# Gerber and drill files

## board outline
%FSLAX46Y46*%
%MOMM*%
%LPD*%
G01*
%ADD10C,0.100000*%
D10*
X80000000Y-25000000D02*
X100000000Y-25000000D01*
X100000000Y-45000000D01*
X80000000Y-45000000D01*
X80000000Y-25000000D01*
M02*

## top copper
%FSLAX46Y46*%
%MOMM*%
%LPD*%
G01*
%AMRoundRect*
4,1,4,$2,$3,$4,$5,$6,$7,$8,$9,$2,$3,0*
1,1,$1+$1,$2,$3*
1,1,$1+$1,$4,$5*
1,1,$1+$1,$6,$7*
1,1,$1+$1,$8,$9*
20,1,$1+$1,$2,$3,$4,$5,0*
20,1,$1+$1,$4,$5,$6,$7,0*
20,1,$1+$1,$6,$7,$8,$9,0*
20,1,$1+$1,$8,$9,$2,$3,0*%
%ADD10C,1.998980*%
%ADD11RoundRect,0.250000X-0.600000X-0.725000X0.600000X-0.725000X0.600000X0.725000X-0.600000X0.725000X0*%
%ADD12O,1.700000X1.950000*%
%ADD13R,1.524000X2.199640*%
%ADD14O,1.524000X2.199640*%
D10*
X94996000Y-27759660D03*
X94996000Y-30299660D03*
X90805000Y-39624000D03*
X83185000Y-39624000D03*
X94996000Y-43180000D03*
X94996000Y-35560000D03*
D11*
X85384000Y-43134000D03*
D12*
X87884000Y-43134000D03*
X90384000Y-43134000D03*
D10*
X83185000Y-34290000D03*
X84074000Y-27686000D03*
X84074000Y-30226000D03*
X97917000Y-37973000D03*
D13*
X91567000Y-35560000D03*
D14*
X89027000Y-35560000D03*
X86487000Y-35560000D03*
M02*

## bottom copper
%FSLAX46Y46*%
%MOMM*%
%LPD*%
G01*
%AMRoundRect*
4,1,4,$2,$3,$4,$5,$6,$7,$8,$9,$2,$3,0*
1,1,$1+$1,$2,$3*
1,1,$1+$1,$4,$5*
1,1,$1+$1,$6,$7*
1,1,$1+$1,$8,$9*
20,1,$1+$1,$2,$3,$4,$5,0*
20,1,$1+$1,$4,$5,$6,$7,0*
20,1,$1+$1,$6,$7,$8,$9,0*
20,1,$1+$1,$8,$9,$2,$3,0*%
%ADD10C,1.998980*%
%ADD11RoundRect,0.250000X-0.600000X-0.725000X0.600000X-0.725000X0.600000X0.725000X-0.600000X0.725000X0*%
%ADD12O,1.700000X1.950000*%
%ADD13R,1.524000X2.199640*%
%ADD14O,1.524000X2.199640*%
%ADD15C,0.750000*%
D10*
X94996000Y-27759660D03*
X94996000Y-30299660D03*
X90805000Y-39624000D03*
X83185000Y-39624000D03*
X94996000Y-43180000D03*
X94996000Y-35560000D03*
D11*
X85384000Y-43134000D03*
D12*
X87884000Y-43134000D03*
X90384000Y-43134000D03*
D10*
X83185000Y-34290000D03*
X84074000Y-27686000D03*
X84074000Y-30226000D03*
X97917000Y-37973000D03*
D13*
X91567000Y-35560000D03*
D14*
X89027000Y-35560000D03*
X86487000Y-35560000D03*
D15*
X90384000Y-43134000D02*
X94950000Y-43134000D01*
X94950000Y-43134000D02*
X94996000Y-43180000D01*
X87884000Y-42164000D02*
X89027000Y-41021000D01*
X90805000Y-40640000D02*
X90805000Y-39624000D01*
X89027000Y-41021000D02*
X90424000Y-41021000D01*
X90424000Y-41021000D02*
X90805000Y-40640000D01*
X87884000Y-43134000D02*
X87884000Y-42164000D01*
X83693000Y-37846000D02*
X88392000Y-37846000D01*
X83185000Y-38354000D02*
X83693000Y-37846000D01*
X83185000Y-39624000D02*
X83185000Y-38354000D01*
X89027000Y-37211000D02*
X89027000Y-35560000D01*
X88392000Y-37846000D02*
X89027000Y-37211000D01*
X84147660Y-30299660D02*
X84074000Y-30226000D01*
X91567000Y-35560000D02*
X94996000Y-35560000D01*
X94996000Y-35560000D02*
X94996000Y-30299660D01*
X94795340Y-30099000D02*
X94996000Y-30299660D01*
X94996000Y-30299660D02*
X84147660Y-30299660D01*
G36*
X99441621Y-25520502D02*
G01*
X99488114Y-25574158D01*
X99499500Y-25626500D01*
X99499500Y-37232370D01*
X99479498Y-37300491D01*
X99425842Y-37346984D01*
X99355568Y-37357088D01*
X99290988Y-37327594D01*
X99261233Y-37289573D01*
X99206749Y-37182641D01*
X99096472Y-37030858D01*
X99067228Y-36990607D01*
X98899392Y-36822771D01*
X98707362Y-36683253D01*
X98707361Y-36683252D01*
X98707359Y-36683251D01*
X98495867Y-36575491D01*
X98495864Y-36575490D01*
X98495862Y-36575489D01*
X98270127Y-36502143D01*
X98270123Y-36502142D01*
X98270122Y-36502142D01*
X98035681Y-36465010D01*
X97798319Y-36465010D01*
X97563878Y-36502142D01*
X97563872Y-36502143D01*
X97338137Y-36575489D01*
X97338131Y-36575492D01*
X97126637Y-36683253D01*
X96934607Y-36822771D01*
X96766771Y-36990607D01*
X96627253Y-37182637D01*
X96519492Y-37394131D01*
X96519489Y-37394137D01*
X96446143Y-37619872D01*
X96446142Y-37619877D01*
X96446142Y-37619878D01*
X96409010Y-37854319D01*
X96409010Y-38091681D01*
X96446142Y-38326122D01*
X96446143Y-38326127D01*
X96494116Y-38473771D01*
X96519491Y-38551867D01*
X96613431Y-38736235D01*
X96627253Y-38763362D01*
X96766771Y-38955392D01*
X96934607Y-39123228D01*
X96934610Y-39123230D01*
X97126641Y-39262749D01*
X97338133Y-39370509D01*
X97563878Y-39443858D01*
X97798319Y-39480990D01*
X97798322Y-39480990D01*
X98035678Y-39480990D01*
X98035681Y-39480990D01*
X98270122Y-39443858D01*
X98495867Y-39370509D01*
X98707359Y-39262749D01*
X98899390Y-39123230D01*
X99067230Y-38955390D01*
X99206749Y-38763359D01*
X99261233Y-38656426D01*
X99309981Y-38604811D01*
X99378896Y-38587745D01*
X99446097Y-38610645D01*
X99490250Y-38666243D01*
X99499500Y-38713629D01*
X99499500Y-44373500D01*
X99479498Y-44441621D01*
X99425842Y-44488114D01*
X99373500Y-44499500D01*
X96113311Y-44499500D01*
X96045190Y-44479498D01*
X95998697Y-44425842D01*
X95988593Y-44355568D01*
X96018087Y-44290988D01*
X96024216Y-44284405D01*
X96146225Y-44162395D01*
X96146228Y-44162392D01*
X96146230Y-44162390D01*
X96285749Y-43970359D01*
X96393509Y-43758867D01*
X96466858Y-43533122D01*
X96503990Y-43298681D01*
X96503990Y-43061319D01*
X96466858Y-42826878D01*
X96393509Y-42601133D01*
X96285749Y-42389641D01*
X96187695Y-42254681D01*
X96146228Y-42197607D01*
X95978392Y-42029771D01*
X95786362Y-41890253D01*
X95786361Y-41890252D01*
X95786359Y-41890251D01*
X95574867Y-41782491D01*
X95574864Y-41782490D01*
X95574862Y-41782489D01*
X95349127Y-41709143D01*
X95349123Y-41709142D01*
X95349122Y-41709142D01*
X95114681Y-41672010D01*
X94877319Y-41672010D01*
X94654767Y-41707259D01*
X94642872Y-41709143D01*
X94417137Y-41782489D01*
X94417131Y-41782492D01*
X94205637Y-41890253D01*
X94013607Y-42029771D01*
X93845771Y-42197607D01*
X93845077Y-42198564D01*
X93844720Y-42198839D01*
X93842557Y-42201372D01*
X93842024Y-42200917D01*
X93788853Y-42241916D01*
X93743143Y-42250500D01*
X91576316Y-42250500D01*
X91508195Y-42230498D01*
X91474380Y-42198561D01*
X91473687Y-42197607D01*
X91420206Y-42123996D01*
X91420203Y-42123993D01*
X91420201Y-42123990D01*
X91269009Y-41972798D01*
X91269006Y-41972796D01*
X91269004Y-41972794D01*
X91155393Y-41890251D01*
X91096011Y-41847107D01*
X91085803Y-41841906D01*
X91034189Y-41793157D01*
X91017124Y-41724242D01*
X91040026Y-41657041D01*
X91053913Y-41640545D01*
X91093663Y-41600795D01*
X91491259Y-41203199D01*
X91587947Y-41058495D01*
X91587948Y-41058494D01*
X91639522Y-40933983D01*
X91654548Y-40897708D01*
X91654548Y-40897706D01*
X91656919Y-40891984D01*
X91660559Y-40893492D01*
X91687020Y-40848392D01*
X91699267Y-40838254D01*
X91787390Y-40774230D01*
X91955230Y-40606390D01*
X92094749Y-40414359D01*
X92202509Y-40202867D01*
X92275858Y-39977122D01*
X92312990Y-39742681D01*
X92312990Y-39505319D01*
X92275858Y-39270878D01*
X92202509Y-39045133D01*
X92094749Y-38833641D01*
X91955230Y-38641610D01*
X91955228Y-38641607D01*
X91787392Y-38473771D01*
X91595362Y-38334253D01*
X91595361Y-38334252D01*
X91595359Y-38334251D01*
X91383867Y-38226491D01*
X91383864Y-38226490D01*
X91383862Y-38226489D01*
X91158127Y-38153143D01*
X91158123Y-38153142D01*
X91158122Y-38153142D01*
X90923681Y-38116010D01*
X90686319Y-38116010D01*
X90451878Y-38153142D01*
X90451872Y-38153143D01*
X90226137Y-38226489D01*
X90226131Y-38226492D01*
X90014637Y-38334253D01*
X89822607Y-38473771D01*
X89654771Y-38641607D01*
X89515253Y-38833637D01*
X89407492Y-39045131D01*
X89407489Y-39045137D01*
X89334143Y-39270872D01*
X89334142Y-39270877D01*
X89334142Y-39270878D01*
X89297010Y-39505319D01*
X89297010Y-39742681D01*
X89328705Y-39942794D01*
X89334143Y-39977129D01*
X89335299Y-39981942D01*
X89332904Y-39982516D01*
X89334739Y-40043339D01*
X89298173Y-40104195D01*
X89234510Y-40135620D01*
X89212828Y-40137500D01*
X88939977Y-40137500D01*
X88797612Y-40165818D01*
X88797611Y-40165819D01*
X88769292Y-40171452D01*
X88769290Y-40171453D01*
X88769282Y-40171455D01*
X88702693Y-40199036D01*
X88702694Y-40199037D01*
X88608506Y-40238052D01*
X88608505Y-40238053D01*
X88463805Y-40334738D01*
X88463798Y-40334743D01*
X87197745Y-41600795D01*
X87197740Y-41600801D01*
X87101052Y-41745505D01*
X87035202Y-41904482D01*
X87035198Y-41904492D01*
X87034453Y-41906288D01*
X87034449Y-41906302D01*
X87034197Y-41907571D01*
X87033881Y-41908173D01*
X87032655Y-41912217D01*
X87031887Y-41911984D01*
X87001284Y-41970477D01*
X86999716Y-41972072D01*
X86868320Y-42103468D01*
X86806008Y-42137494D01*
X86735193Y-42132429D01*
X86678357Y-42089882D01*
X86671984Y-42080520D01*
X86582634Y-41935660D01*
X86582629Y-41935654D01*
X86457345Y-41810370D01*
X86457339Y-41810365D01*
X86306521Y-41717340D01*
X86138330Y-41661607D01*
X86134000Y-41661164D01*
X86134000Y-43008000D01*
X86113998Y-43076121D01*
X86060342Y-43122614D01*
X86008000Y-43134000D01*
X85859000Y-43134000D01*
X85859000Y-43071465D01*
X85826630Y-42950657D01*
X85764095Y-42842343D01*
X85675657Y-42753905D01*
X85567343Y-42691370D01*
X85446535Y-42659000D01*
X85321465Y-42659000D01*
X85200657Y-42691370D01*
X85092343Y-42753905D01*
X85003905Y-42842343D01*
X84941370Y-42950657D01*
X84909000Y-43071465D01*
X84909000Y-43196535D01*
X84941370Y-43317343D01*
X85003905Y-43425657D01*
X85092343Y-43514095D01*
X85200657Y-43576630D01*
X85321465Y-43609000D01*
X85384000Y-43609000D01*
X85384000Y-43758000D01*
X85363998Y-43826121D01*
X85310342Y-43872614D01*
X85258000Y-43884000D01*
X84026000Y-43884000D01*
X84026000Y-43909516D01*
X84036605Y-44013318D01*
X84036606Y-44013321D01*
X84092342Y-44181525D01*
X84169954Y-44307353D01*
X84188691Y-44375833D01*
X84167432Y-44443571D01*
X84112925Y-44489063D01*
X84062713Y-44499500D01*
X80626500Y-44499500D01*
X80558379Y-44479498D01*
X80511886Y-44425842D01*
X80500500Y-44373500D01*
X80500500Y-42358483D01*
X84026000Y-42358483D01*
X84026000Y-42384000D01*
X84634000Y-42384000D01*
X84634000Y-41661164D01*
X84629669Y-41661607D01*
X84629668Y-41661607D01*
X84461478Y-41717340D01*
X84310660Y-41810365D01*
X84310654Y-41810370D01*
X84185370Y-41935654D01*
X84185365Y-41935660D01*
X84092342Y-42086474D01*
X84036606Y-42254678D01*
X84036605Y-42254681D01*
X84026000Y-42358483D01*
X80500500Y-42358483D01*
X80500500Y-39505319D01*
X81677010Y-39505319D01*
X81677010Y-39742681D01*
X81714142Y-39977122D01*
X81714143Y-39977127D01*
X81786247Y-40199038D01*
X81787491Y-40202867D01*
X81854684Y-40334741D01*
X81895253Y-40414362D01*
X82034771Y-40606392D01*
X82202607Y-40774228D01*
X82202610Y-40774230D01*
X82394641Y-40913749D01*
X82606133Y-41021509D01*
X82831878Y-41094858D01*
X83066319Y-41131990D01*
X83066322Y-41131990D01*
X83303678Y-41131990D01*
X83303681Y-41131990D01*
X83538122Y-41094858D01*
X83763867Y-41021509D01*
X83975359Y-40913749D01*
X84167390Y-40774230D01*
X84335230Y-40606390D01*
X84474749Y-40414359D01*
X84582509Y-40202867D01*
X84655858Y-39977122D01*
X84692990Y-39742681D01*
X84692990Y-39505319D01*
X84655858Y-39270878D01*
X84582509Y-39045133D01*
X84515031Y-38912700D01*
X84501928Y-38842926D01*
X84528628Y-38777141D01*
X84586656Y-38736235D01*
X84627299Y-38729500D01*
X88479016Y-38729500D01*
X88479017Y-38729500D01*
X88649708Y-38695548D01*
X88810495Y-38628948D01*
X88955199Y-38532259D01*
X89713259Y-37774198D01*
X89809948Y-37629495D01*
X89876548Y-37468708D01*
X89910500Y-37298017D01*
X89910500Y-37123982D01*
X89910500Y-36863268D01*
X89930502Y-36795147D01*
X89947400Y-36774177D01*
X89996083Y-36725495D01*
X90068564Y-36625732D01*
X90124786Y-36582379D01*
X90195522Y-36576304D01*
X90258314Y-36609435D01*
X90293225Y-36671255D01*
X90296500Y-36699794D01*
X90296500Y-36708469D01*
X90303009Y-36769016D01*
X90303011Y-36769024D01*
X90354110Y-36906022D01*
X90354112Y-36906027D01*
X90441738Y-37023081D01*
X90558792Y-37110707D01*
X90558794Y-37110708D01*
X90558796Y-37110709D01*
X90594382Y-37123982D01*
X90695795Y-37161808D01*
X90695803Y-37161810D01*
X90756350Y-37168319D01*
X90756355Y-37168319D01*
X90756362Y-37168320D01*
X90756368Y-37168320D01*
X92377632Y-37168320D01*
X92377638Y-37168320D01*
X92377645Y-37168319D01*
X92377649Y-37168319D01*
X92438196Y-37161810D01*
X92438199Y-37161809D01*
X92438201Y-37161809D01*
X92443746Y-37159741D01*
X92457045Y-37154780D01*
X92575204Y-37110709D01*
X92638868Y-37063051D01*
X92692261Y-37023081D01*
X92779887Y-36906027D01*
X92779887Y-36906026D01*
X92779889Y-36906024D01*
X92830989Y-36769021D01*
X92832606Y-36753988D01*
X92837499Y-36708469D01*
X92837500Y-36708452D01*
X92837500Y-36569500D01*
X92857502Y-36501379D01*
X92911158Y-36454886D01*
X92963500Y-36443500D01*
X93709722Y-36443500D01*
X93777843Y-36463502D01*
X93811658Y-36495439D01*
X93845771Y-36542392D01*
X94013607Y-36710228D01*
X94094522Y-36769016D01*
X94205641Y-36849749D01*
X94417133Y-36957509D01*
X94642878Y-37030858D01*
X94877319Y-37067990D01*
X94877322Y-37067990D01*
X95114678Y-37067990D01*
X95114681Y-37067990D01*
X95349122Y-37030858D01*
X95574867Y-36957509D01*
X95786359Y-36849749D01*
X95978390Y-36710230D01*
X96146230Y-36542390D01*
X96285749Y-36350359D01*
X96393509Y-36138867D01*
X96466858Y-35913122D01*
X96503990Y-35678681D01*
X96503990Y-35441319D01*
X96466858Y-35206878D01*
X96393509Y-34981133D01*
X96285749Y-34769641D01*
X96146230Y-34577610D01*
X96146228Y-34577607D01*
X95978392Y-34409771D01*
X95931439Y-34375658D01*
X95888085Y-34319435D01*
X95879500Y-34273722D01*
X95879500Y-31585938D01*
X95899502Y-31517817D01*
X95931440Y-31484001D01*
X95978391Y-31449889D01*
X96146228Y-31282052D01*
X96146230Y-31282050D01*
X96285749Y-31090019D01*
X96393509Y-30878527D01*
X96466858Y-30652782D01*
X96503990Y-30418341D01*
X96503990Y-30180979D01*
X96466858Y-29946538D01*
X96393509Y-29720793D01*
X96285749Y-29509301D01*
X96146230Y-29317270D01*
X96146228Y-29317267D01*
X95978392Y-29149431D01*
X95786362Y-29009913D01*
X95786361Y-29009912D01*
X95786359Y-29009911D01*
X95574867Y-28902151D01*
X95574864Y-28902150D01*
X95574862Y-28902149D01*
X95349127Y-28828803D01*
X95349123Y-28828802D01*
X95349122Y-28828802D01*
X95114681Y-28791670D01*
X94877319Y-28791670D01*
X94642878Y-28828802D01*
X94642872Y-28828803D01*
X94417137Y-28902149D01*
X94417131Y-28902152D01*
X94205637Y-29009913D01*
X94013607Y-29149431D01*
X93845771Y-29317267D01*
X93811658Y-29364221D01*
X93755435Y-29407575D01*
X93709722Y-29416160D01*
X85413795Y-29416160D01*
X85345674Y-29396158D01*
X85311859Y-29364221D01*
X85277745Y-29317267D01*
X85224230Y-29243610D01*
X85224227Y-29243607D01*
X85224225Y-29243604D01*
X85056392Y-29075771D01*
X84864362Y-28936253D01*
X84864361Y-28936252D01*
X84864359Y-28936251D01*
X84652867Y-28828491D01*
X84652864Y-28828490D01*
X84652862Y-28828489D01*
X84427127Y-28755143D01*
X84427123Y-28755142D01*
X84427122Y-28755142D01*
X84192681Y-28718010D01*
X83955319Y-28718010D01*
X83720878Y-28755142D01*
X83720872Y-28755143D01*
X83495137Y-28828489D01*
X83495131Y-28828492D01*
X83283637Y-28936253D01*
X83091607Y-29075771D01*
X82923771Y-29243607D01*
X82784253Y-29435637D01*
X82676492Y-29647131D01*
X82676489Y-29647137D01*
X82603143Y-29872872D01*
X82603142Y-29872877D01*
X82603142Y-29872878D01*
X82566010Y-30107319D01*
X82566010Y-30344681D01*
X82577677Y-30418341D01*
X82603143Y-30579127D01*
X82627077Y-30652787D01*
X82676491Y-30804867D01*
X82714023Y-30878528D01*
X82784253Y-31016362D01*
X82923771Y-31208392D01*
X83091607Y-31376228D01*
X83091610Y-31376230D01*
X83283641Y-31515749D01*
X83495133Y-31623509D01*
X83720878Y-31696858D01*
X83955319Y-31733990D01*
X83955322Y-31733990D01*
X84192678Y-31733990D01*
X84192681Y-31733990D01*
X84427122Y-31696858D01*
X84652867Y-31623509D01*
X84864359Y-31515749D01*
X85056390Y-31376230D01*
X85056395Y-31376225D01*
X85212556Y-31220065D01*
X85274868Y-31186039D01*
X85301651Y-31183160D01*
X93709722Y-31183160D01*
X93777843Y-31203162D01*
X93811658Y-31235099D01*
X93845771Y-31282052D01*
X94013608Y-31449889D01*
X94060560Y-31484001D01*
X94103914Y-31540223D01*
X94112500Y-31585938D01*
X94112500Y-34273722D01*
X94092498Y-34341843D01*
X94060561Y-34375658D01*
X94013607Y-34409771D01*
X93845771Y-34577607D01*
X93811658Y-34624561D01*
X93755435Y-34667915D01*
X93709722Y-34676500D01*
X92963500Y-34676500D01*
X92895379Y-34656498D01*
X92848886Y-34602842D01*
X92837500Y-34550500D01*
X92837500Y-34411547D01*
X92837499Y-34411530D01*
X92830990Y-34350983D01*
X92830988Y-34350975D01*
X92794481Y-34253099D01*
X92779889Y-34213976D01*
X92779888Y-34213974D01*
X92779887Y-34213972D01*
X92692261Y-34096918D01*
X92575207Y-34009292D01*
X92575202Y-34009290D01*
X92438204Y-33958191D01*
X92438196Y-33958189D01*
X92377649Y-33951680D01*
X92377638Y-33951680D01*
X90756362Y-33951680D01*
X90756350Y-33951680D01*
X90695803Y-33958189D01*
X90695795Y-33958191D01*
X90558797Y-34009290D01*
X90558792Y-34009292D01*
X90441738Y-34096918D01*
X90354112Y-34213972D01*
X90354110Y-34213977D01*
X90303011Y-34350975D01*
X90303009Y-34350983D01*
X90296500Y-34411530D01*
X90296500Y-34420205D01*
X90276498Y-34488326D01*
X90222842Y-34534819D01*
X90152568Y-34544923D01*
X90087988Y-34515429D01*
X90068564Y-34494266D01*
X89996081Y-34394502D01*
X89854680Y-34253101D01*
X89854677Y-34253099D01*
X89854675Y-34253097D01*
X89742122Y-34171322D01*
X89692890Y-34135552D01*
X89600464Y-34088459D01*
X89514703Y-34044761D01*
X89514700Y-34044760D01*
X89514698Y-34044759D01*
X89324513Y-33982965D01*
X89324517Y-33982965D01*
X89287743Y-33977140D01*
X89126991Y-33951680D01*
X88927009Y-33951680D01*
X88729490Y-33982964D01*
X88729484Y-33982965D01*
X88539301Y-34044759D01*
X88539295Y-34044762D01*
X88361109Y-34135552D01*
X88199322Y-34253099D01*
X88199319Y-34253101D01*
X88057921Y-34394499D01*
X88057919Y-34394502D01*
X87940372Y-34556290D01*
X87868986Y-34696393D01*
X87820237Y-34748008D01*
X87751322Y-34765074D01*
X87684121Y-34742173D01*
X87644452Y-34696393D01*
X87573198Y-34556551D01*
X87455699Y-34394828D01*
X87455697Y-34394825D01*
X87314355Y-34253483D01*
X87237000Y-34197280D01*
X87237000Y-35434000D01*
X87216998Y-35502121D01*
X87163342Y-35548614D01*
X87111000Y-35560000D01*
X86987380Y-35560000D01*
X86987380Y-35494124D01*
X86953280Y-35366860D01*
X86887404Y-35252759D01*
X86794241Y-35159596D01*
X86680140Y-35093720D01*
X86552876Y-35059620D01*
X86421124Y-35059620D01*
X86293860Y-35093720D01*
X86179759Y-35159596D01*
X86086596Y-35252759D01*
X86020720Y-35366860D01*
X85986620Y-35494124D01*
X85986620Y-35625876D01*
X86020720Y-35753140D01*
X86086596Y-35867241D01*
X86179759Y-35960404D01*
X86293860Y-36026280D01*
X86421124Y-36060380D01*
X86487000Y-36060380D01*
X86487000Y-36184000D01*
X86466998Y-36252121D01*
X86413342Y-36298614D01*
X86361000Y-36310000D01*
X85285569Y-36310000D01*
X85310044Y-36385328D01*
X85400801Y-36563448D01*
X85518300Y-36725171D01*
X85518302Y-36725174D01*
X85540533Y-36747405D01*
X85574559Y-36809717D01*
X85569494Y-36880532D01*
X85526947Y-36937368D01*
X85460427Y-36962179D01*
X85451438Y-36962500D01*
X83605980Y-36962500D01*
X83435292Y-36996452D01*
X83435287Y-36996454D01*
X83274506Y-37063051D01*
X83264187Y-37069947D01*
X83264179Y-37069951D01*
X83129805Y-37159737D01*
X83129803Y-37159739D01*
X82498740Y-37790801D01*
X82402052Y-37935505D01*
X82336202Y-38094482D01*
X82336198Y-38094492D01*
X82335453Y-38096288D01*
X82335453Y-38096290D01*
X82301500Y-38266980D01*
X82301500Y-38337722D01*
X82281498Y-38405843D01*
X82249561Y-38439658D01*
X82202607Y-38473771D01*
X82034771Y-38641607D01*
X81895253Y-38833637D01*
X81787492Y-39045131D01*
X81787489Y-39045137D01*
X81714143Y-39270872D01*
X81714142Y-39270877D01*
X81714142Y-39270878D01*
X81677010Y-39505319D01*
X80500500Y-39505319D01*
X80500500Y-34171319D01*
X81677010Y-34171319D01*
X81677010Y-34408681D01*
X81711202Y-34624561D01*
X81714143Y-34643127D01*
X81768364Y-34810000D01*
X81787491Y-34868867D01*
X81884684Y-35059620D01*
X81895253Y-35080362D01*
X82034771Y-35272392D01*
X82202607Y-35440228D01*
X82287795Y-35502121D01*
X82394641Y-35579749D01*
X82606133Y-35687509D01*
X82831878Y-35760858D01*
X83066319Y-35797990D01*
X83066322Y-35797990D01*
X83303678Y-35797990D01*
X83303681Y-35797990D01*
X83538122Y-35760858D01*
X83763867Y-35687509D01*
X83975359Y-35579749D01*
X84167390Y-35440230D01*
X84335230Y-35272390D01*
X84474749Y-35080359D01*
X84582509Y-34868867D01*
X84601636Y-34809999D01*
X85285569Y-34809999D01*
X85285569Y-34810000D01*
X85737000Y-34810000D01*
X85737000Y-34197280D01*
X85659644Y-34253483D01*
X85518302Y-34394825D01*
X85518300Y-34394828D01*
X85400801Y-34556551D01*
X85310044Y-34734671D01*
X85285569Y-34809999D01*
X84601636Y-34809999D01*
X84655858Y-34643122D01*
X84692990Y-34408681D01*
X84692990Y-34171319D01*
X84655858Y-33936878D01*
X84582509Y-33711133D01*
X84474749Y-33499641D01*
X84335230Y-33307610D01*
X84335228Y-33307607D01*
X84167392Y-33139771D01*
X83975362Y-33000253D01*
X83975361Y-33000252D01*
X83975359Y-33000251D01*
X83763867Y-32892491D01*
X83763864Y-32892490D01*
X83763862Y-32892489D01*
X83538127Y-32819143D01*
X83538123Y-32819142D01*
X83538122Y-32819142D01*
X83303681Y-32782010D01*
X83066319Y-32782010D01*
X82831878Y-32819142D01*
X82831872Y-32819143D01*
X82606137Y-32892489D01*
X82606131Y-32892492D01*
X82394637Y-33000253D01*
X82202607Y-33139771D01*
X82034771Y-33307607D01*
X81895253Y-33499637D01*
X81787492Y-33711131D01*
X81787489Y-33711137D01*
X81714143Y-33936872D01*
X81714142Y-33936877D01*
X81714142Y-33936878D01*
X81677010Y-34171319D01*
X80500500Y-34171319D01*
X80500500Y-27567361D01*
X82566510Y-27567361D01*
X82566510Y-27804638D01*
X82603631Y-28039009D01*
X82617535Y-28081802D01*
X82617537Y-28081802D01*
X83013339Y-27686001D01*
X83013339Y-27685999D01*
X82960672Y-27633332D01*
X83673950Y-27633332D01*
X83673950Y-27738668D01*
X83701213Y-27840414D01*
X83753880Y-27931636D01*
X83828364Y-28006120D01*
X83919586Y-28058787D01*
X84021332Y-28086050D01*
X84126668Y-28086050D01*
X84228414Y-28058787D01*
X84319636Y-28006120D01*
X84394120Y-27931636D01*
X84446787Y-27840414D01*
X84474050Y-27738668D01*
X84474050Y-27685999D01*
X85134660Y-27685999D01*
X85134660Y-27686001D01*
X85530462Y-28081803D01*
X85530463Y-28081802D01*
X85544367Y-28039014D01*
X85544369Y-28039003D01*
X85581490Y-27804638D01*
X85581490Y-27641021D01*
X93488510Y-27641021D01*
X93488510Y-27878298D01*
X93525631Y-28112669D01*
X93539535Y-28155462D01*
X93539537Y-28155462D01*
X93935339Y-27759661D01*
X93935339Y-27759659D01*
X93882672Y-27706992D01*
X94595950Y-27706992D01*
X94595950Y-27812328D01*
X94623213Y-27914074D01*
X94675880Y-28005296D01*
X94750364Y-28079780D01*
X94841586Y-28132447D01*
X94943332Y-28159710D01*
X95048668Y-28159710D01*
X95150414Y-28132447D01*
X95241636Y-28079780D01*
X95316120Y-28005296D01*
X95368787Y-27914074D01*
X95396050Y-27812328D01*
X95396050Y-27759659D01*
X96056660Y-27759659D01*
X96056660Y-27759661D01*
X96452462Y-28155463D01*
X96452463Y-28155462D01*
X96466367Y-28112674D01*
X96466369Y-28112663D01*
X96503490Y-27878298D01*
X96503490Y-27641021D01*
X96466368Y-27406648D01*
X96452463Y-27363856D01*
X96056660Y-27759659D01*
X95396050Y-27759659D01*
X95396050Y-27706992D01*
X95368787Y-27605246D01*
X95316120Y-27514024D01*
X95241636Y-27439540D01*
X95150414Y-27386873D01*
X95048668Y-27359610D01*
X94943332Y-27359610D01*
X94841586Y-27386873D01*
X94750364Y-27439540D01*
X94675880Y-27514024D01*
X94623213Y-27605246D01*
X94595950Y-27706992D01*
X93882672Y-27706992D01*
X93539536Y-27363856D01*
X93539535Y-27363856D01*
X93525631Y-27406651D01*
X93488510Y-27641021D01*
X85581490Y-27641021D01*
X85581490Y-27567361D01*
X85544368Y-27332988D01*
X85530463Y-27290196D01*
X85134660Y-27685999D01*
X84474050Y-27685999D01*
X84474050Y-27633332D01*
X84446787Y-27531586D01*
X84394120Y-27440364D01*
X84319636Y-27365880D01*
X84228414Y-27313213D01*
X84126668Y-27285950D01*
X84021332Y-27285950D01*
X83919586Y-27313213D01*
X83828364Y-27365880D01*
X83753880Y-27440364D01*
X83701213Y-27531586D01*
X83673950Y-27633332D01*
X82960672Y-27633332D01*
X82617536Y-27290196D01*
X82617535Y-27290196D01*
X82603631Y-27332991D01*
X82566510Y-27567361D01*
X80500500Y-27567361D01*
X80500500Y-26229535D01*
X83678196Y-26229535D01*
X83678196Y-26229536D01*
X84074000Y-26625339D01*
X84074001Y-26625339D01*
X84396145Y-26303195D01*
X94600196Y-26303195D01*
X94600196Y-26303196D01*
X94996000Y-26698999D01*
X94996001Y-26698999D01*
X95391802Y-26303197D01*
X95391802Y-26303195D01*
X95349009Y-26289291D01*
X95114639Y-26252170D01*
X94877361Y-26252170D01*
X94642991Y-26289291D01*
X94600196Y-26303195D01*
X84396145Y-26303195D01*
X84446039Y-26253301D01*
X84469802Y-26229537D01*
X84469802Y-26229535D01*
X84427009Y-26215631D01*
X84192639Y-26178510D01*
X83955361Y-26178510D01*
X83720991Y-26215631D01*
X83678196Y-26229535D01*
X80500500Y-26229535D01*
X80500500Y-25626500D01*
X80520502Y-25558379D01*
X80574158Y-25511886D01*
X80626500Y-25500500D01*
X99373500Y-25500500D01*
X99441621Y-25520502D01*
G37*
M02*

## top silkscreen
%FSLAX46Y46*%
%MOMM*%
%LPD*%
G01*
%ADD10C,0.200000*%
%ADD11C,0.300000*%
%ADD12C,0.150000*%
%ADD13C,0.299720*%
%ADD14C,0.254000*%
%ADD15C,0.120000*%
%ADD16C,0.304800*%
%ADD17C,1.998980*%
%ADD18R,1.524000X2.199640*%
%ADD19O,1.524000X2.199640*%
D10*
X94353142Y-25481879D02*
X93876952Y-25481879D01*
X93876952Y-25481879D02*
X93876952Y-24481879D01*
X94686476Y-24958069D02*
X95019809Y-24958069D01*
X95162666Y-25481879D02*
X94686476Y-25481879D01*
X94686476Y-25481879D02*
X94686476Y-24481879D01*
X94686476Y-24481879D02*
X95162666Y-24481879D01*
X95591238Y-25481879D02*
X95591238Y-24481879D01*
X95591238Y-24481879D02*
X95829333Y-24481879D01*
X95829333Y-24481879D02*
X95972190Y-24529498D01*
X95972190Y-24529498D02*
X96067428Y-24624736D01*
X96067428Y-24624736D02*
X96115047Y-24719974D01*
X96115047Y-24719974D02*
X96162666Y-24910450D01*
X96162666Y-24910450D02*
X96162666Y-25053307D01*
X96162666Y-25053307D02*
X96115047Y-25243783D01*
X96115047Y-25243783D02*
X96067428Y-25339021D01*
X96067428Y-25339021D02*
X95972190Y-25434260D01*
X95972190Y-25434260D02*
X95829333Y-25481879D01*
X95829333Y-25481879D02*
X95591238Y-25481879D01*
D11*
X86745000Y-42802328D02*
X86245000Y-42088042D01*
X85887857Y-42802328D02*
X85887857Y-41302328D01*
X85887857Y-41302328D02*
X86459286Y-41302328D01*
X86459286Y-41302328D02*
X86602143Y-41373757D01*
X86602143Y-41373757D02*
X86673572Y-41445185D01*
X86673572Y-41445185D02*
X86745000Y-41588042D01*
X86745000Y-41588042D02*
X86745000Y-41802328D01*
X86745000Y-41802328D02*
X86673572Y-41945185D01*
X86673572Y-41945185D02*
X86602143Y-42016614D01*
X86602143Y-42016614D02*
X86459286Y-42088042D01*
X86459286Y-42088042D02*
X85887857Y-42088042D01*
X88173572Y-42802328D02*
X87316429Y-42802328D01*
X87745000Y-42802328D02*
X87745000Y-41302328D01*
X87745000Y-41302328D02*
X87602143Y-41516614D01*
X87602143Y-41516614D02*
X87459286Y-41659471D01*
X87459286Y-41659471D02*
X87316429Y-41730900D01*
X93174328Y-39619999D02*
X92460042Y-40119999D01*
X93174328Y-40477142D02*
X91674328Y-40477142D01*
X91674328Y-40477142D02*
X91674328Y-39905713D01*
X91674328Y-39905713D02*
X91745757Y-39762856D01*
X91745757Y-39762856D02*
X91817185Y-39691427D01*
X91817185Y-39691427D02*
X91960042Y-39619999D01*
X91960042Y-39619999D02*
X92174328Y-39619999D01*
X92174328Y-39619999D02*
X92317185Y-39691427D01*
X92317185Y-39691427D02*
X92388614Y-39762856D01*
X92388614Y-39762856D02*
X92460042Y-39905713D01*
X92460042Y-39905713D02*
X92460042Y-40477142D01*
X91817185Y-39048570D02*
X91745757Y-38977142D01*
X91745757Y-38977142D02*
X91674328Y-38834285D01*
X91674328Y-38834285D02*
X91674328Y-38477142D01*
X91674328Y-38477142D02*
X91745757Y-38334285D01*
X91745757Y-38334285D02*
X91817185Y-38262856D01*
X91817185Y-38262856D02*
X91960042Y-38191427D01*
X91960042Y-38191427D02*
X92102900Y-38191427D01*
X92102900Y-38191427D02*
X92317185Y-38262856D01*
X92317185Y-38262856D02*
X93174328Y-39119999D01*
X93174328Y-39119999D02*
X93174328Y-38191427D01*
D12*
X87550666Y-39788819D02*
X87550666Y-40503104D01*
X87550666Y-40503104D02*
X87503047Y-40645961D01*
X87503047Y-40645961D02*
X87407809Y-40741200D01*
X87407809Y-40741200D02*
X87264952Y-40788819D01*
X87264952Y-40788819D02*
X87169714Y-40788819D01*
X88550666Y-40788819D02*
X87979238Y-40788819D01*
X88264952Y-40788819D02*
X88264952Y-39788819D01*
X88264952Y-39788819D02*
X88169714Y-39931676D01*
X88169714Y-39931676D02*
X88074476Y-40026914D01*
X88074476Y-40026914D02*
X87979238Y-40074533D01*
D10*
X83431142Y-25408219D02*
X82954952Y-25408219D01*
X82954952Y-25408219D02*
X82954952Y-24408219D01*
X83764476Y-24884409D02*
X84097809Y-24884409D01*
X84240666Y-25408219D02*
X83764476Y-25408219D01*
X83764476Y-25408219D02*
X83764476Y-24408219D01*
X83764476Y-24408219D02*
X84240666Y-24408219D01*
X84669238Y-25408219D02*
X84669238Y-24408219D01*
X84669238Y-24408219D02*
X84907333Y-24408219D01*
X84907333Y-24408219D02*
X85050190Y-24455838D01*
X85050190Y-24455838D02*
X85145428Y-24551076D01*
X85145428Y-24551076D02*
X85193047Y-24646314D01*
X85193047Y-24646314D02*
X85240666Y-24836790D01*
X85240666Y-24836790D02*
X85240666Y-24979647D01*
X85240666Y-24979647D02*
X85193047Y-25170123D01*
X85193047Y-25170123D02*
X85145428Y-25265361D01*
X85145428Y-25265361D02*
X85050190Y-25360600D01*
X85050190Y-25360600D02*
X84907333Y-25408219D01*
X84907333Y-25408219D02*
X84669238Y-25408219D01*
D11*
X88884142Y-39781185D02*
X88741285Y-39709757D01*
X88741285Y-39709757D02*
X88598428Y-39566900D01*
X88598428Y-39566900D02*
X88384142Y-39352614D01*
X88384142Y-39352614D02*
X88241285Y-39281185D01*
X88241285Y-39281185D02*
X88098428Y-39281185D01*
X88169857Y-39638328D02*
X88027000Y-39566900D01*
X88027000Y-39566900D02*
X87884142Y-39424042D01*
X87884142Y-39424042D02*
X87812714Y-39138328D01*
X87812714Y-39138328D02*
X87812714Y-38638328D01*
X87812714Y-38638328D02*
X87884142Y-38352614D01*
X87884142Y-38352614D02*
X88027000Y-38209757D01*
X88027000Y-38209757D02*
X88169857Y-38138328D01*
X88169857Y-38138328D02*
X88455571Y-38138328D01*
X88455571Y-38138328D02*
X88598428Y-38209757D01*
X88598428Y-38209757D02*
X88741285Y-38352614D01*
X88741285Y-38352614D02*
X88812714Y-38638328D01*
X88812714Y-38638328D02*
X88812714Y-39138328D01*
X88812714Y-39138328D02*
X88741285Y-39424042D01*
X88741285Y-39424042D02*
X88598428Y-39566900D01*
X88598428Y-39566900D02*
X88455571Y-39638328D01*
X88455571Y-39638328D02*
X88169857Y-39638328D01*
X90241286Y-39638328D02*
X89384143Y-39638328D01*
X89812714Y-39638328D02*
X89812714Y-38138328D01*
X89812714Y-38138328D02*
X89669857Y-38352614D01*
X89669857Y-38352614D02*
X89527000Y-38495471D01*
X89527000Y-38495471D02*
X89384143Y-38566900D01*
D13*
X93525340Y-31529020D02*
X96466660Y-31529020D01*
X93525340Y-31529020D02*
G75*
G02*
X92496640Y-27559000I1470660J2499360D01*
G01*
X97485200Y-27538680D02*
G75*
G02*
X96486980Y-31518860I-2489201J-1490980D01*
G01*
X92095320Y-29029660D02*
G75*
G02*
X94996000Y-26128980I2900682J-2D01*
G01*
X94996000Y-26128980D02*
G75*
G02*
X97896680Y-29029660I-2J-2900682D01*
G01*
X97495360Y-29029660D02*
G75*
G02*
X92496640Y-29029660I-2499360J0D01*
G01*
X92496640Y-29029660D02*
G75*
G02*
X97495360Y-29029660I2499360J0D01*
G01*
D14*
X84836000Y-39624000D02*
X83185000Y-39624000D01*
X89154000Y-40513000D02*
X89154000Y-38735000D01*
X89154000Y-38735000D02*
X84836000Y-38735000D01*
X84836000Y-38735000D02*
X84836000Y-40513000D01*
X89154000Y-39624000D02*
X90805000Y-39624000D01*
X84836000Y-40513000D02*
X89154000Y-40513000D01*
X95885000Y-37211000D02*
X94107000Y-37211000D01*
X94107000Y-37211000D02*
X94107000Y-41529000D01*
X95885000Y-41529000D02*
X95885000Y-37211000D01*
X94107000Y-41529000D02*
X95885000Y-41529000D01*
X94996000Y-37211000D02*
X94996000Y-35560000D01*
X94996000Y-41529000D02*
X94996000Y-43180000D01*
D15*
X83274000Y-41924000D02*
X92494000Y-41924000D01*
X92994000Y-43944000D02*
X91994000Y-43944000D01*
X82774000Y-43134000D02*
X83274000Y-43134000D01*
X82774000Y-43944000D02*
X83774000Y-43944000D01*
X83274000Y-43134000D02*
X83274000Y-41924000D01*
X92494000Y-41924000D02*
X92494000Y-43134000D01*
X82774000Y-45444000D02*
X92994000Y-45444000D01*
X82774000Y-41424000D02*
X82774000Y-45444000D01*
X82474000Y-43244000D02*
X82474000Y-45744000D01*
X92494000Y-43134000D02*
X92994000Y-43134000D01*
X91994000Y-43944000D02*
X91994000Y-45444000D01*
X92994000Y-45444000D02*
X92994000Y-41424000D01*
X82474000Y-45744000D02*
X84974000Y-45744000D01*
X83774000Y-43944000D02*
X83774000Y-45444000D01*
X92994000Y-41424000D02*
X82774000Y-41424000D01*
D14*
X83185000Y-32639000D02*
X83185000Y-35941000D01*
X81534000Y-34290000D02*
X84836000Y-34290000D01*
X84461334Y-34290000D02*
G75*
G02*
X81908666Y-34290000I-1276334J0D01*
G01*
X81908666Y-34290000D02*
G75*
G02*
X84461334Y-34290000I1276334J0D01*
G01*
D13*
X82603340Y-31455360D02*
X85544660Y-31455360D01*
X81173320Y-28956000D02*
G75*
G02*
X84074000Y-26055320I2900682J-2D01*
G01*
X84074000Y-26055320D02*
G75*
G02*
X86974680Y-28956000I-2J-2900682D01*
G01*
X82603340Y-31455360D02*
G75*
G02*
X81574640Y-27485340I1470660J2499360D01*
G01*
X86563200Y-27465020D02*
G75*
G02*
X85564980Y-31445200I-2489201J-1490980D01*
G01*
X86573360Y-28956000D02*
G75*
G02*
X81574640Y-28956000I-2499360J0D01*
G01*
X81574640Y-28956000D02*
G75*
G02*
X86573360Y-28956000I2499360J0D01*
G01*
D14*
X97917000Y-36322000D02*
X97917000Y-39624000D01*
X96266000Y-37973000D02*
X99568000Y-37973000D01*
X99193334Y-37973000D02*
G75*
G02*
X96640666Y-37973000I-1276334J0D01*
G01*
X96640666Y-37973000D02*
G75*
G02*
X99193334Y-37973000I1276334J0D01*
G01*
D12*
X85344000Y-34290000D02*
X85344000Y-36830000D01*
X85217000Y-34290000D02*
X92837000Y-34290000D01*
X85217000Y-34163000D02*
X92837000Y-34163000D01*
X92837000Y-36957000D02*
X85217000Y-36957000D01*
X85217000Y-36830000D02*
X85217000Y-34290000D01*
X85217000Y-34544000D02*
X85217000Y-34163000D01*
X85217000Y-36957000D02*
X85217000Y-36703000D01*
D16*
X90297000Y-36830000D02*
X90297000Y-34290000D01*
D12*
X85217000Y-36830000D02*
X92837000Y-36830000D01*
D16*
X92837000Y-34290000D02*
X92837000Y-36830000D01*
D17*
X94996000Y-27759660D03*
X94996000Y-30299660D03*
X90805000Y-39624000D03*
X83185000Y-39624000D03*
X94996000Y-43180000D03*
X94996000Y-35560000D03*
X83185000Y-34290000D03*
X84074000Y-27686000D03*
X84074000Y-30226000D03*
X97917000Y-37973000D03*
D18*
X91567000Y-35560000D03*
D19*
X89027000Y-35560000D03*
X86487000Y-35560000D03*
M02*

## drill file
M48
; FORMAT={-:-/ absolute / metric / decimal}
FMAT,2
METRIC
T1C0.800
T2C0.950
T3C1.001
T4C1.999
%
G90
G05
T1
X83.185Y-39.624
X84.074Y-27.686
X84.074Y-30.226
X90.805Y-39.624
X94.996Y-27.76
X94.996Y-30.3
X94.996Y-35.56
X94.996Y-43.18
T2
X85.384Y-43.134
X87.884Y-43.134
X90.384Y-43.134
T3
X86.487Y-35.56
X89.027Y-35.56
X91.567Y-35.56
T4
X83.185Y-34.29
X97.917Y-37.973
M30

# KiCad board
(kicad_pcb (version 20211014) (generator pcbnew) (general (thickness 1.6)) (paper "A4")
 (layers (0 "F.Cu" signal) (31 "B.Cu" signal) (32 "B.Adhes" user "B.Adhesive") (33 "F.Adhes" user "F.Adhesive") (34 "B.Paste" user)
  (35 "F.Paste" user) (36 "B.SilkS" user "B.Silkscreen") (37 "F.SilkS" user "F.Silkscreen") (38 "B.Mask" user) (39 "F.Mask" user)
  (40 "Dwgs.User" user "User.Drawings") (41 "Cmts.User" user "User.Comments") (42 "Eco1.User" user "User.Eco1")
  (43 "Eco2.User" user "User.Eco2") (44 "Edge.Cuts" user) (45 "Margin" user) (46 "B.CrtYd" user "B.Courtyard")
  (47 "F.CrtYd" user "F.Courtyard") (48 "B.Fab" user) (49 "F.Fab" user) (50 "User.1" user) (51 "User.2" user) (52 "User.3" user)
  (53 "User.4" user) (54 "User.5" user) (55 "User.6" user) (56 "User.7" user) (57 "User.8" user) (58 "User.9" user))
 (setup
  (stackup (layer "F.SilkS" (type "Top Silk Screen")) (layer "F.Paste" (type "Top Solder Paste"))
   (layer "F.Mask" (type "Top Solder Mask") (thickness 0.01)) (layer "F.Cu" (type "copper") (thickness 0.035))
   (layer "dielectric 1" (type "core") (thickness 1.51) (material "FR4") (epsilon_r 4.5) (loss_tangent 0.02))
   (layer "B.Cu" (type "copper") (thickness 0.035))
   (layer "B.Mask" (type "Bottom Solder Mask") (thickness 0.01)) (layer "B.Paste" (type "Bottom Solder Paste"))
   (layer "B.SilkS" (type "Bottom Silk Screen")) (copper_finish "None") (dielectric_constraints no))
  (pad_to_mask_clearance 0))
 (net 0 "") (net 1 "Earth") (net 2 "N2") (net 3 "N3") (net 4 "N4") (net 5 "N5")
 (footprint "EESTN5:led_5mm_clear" (layer "F.Cu") (at 94.996 29.02966)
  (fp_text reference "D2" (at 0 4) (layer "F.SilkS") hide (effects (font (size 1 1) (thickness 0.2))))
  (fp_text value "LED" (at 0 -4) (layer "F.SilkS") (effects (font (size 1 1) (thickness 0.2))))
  (fp_line (start -1.47066 2.49936) (end 1.47066 2.49936) (layer "F.SilkS") (width 0.29972))
  (fp_arc (start -1.47066 2.49936) (mid -2.807228 0.727401) (end -2.49936 -1.47066) (layer "F.SilkS") (width 0.29972))
  (fp_arc (start 2.4892 -1.49098) (mid 2.814412 0.705848) (end 1.49098 2.4892) (layer "F.SilkS") (width 0.29972))
  (fp_arc (start -2.90068 0) (mid -2.05109 -2.05109) (end 0 -2.90068) (layer "F.SilkS") (width 0.29972))
  (fp_arc (start 0 -2.90068) (mid 2.05109 -2.05109) (end 2.90068 0) (layer "F.SilkS") (width 0.29972))
  (fp_circle (center 0 0) (end -2.49936 0) (layer "F.SilkS") (width 0.29972) (fill none))
  (pad "1" thru_hole circle locked (at 0 -1.27) (size 1.99898 1.99898) (drill 0.8001) (layers *.Cu *.Mask "F.SilkS") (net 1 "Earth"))
  (pad "2" thru_hole circle locked (at 0 1.27) (size 1.99898 1.99898) (drill 0.8001) (layers *.Cu *.Mask "F.SilkS") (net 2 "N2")))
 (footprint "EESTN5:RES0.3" (layer "F.Cu") (at 86.995 39.624 180) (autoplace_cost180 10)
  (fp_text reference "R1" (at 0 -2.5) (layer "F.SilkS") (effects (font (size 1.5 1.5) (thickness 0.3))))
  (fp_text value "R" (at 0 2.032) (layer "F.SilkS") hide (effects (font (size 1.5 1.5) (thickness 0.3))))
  (fp_line (start 2.159 0) (end 3.81 0) (layer "F.SilkS") (width 0.254))
  (fp_line (start -2.159 -0.889) (end -2.159 0.889) (layer "F.SilkS") (width 0.254))
  (fp_line (start -2.159 0.889) (end 2.159 0.889) (layer "F.SilkS") (width 0.254))
  (fp_line (start 2.159 0.889) (end 2.159 -0.889) (layer "F.SilkS") (width 0.254))
  (fp_line (start -2.159 0) (end -3.81 0) (layer "F.SilkS") (width 0.254))
  (fp_line (start 2.159 -0.889) (end -2.159 -0.889) (layer "F.SilkS") (width 0.254))
  (pad "1" thru_hole circle locked (at -3.81 0 180) (size 1.99898 1.99898) (drill 0.8001) (layers *.Cu *.Mask "F.SilkS") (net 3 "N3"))
  (pad "2" thru_hole circle locked (at 3.81 0 180) (size 1.99898 1.99898) (drill 0.8001) (layers *.Cu *.Mask "F.SilkS") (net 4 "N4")))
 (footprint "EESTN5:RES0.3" (layer "F.Cu") (at 94.996 39.37 90) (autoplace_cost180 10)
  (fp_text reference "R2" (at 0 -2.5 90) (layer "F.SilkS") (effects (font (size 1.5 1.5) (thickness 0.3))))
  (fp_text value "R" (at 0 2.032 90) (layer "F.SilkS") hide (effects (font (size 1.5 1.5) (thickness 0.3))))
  (fp_line (start 2.159 0.889) (end 2.159 -0.889) (layer "F.SilkS") (width 0.254))
  (fp_line (start 2.159 -0.889) (end -2.159 -0.889) (layer "F.SilkS") (width 0.254))
  (fp_line (start -2.159 0.889) (end 2.159 0.889) (layer "F.SilkS") (width 0.254))
  (fp_line (start -2.159 -0.889) (end -2.159 0.889) (layer "F.SilkS") (width 0.254))
  (fp_line (start 2.159 0) (end 3.81 0) (layer "F.SilkS") (width 0.254))
  (fp_line (start -2.159 0) (end -3.81 0) (layer "F.SilkS") (width 0.254))
  (pad "1" thru_hole circle locked (at -3.81 0 90) (size 1.99898 1.99898) (drill 0.8001) (layers *.Cu *.Mask "F.SilkS") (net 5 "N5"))
  (pad "2" thru_hole circle locked (at 3.81 0 90) (size 1.99898 1.99898) (drill 0.8001) (layers *.Cu *.Mask "F.SilkS") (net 2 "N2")))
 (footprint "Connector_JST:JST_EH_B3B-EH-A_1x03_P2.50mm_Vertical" (layer "F.Cu") (at 85.384 43.134)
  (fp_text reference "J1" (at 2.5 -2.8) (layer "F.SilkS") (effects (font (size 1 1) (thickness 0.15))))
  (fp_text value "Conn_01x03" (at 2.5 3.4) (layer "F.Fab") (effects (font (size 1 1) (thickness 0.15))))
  (fp_line (start -2.11 -1.21) (end 7.11 -1.21) (layer "F.SilkS") (width 0.12))
  (fp_line (start 7.61 0.81) (end 6.61 0.81) (layer "F.SilkS") (width 0.12))
  (fp_line (start -2.61 0) (end -2.11 0) (layer "F.SilkS") (width 0.12))
  (fp_line (start -2.61 0.81) (end -1.61 0.81) (layer "F.SilkS") (width 0.12))
  (fp_line (start -2.11 0) (end -2.11 -1.21) (layer "F.SilkS") (width 0.12))
  (fp_line (start 7.11 -1.21) (end 7.11 0) (layer "F.SilkS") (width 0.12))
  (fp_line (start -2.61 2.31) (end 7.61 2.31) (layer "F.SilkS") (width 0.12))
  (fp_line (start -2.61 -1.71) (end -2.61 2.31) (layer "F.SilkS") (width 0.12))
  (fp_line (start -2.91 0.11) (end -2.91 2.61) (layer "F.SilkS") (width 0.12))
  (fp_line (start 7.11 0) (end 7.61 0) (layer "F.SilkS") (width 0.12))
  (fp_line (start 6.61 0.81) (end 6.61 2.31) (layer "F.SilkS") (width 0.12))
  (fp_line (start 7.61 2.31) (end 7.61 -1.71) (layer "F.SilkS") (width 0.12))
  (fp_line (start -2.91 2.61) (end -0.41 2.61) (layer "F.SilkS") (width 0.12))
  (fp_line (start -1.61 0.81) (end -1.61 2.31) (layer "F.SilkS") (width 0.12))
  (fp_line (start 7.61 -1.71) (end -2.61 -1.71) (layer "F.SilkS") (width 0.12))
  (pad "1" thru_hole roundrect (at 0 0) (size 1.7 1.95) (drill 0.95) (layers *.Cu *.Mask) (roundrect_rratio 0.1470588235) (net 1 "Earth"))
  (pad "2" thru_hole oval (at 2.5 0) (size 1.7 1.95) (drill 0.95) (layers *.Cu *.Mask) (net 3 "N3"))
  (pad "3" thru_hole oval (at 5 0) (size 1.7 1.95) (drill 0.95) (layers *.Cu *.Mask) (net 5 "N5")))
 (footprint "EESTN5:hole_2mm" (layer "F.Cu") (at 83.185 34.29)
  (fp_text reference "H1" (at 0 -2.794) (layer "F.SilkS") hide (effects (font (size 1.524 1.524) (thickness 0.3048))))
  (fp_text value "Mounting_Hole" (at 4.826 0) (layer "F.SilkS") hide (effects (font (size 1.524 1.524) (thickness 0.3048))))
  (fp_line (start 0 -1.651) (end 0 1.651) (layer "F.SilkS") (width 0.254))
  (fp_line (start -1.651 0) (end 1.651 0) (layer "F.SilkS") (width 0.254))
  (fp_circle (center 0 0) (end 1.27 -0.127) (layer "F.SilkS") (width 0.254) (fill none))
  (pad "1" thru_hole circle locked (at 0 0) (size 1.99898 1.99898) (drill 1.99898) (layers *.Cu "F.SilkS")))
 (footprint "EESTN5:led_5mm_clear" (layer "F.Cu") (at 84.074 28.956)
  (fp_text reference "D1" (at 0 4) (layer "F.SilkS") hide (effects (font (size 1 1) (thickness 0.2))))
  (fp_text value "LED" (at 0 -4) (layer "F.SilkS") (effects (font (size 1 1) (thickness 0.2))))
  (fp_line (start -1.47066 2.49936) (end 1.47066 2.49936) (layer "F.SilkS") (width 0.29972))
  (fp_arc (start -2.90068 0) (mid -2.05109 -2.05109) (end 0 -2.90068) (layer "F.SilkS") (width 0.29972))
  (fp_arc (start 0 -2.90068) (mid 2.05109 -2.05109) (end 2.90068 0) (layer "F.SilkS") (width 0.29972))
  (fp_arc (start -1.47066 2.49936) (mid -2.807228 0.727401) (end -2.49936 -1.47066) (layer "F.SilkS") (width 0.29972))
  (fp_arc (start 2.4892 -1.49098) (mid 2.814412 0.705848) (end 1.49098 2.4892) (layer "F.SilkS") (width 0.29972))
  (fp_circle (center 0 0) (end -2.49936 0) (layer "F.SilkS") (width 0.29972) (fill none))
  (pad "1" thru_hole circle locked (at 0 -1.27) (size 1.99898 1.99898) (drill 0.8001) (layers *.Cu *.Mask "F.SilkS") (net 1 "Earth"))
  (pad "2" thru_hole circle locked (at 0 1.27) (size 1.99898 1.99898) (drill 0.8001) (layers *.Cu *.Mask "F.SilkS") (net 2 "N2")))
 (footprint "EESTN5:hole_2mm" (layer "F.Cu") (at 97.917 37.973)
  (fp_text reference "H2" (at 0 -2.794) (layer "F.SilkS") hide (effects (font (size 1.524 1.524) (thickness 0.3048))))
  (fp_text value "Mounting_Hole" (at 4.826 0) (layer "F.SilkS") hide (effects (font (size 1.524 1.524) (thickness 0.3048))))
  (fp_line (start 0 -1.651) (end 0 1.651) (layer "F.SilkS") (width 0.254))
  (fp_line (start -1.651 0) (end 1.651 0) (layer "F.SilkS") (width 0.254))
  (fp_circle (center 0 0) (end 1.27 -0.127) (layer "F.SilkS") (width 0.254) (fill none))
  (pad "1" thru_hole circle locked (at 0 0) (size 1.99898 1.99898) (drill 1.99898) (layers *.Cu "F.SilkS")))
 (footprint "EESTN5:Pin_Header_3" (layer "F.Cu") (at 89.027 35.56 180)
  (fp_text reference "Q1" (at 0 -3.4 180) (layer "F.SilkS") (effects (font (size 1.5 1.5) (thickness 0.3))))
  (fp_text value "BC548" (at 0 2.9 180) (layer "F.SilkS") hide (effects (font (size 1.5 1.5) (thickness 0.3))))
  (fp_line (start 3.683 1.27) (end 3.683 -1.27) (layer "F.SilkS") (width 0.15))
  (fp_line (start 3.81 1.27) (end -3.81 1.27) (layer "F.SilkS") (width 0.15))
  (fp_line (start 3.81 1.397) (end -3.81 1.397) (layer "F.SilkS") (width 0.15))
  (fp_line (start -3.81 -1.397) (end 3.81 -1.397) (layer "F.SilkS") (width 0.15))
  (fp_line (start 3.81 -1.27) (end 3.81 1.27) (layer "F.SilkS") (width 0.15))
  (fp_line (start 3.81 1.016) (end 3.81 1.397) (layer "F.SilkS") (width 0.15))
  (fp_line (start 3.81 -1.397) (end 3.81 -1.143) (layer "F.SilkS") (width 0.15))
  (fp_line (start -1.27 -1.27) (end -1.27 1.27) (layer "F.SilkS") (width 0.3048))
  (fp_line (start 3.81 -1.27) (end -3.81 -1.27) (layer "F.SilkS") (width 0.15))
  (fp_line (start -3.81 1.27) (end -3.81 -1.27) (layer "F.SilkS") (width 0.3048))
  (pad "1" thru_hole rect locked (at -2.54 0 180) (size 1.524 2.19964) (drill 1.00076) (layers *.Cu *.Mask "F.SilkS") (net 2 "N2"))
  (pad "2" thru_hole oval locked (at 0 0 180) (size 1.524 2.19964) (drill 1.00076) (layers *.Cu *.Mask "F.SilkS") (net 4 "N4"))
  (pad "3" thru_hole oval locked (at 2.54 0 180) (size 1.524 2.19964) (drill 1.00076) (layers *.Cu *.Mask "F.SilkS") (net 1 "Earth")))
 (gr_rect (start 80 25) (end 100 45) (layer "Edge.Cuts") (width 0.1) (fill none))
 (segment (start 90.384 43.134) (end 94.95 43.134) (width 0.75) (layer "B.Cu") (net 5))
 (segment (start 94.95 43.134) (end 94.996 43.18) (width 0.75) (layer "B.Cu") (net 5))
 (segment (start 87.884 42.164) (end 89.027 41.021) (width 0.75) (layer "B.Cu") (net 3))
 (segment (start 90.805 40.64) (end 90.805 39.624) (width 0.75) (layer "B.Cu") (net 3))
 (segment (start 89.027 41.021) (end 90.424 41.021) (width 0.75) (layer "B.Cu") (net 3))
 (segment (start 90.424 41.021) (end 90.805 40.64) (width 0.75) (layer "B.Cu") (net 3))
 (segment (start 87.884 43.134) (end 87.884 42.164) (width 0.75) (layer "B.Cu") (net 3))
 (segment (start 83.693 37.846) (end 88.392 37.846) (width 0.75) (layer "B.Cu") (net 4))
 (segment (start 83.185 38.354) (end 83.693 37.846) (width 0.75) (layer "B.Cu") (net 4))
 (segment (start 83.185 39.624) (end 83.185 38.354) (width 0.75) (layer "B.Cu") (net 4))
 (segment (start 89.027 37.211) (end 89.027 35.56) (width 0.75) (layer "B.Cu") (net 4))
 (segment (start 88.392 37.846) (end 89.027 37.211) (width 0.75) (layer "B.Cu") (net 4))
 (segment (start 84.14766 30.29966) (end 84.074 30.226) (width 0.75) (layer "B.Cu") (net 2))
 (segment (start 91.567 35.56) (end 94.996 35.56) (width 0.75) (layer "B.Cu") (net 2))
 (segment (start 94.996 35.56) (end 94.996 30.29966) (width 0.75) (layer "B.Cu") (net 2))
 (segment (start 94.79534 30.099) (end 94.996 30.29966) (width 0.75) (layer "B.Cu") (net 2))
 (segment (start 94.996 30.29966) (end 84.14766 30.29966) (width 0.75) (layer "B.Cu") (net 2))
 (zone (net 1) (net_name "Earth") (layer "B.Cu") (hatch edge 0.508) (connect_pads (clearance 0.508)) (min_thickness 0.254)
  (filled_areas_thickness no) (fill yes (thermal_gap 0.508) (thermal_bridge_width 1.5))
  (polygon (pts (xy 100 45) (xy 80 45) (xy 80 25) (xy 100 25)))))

